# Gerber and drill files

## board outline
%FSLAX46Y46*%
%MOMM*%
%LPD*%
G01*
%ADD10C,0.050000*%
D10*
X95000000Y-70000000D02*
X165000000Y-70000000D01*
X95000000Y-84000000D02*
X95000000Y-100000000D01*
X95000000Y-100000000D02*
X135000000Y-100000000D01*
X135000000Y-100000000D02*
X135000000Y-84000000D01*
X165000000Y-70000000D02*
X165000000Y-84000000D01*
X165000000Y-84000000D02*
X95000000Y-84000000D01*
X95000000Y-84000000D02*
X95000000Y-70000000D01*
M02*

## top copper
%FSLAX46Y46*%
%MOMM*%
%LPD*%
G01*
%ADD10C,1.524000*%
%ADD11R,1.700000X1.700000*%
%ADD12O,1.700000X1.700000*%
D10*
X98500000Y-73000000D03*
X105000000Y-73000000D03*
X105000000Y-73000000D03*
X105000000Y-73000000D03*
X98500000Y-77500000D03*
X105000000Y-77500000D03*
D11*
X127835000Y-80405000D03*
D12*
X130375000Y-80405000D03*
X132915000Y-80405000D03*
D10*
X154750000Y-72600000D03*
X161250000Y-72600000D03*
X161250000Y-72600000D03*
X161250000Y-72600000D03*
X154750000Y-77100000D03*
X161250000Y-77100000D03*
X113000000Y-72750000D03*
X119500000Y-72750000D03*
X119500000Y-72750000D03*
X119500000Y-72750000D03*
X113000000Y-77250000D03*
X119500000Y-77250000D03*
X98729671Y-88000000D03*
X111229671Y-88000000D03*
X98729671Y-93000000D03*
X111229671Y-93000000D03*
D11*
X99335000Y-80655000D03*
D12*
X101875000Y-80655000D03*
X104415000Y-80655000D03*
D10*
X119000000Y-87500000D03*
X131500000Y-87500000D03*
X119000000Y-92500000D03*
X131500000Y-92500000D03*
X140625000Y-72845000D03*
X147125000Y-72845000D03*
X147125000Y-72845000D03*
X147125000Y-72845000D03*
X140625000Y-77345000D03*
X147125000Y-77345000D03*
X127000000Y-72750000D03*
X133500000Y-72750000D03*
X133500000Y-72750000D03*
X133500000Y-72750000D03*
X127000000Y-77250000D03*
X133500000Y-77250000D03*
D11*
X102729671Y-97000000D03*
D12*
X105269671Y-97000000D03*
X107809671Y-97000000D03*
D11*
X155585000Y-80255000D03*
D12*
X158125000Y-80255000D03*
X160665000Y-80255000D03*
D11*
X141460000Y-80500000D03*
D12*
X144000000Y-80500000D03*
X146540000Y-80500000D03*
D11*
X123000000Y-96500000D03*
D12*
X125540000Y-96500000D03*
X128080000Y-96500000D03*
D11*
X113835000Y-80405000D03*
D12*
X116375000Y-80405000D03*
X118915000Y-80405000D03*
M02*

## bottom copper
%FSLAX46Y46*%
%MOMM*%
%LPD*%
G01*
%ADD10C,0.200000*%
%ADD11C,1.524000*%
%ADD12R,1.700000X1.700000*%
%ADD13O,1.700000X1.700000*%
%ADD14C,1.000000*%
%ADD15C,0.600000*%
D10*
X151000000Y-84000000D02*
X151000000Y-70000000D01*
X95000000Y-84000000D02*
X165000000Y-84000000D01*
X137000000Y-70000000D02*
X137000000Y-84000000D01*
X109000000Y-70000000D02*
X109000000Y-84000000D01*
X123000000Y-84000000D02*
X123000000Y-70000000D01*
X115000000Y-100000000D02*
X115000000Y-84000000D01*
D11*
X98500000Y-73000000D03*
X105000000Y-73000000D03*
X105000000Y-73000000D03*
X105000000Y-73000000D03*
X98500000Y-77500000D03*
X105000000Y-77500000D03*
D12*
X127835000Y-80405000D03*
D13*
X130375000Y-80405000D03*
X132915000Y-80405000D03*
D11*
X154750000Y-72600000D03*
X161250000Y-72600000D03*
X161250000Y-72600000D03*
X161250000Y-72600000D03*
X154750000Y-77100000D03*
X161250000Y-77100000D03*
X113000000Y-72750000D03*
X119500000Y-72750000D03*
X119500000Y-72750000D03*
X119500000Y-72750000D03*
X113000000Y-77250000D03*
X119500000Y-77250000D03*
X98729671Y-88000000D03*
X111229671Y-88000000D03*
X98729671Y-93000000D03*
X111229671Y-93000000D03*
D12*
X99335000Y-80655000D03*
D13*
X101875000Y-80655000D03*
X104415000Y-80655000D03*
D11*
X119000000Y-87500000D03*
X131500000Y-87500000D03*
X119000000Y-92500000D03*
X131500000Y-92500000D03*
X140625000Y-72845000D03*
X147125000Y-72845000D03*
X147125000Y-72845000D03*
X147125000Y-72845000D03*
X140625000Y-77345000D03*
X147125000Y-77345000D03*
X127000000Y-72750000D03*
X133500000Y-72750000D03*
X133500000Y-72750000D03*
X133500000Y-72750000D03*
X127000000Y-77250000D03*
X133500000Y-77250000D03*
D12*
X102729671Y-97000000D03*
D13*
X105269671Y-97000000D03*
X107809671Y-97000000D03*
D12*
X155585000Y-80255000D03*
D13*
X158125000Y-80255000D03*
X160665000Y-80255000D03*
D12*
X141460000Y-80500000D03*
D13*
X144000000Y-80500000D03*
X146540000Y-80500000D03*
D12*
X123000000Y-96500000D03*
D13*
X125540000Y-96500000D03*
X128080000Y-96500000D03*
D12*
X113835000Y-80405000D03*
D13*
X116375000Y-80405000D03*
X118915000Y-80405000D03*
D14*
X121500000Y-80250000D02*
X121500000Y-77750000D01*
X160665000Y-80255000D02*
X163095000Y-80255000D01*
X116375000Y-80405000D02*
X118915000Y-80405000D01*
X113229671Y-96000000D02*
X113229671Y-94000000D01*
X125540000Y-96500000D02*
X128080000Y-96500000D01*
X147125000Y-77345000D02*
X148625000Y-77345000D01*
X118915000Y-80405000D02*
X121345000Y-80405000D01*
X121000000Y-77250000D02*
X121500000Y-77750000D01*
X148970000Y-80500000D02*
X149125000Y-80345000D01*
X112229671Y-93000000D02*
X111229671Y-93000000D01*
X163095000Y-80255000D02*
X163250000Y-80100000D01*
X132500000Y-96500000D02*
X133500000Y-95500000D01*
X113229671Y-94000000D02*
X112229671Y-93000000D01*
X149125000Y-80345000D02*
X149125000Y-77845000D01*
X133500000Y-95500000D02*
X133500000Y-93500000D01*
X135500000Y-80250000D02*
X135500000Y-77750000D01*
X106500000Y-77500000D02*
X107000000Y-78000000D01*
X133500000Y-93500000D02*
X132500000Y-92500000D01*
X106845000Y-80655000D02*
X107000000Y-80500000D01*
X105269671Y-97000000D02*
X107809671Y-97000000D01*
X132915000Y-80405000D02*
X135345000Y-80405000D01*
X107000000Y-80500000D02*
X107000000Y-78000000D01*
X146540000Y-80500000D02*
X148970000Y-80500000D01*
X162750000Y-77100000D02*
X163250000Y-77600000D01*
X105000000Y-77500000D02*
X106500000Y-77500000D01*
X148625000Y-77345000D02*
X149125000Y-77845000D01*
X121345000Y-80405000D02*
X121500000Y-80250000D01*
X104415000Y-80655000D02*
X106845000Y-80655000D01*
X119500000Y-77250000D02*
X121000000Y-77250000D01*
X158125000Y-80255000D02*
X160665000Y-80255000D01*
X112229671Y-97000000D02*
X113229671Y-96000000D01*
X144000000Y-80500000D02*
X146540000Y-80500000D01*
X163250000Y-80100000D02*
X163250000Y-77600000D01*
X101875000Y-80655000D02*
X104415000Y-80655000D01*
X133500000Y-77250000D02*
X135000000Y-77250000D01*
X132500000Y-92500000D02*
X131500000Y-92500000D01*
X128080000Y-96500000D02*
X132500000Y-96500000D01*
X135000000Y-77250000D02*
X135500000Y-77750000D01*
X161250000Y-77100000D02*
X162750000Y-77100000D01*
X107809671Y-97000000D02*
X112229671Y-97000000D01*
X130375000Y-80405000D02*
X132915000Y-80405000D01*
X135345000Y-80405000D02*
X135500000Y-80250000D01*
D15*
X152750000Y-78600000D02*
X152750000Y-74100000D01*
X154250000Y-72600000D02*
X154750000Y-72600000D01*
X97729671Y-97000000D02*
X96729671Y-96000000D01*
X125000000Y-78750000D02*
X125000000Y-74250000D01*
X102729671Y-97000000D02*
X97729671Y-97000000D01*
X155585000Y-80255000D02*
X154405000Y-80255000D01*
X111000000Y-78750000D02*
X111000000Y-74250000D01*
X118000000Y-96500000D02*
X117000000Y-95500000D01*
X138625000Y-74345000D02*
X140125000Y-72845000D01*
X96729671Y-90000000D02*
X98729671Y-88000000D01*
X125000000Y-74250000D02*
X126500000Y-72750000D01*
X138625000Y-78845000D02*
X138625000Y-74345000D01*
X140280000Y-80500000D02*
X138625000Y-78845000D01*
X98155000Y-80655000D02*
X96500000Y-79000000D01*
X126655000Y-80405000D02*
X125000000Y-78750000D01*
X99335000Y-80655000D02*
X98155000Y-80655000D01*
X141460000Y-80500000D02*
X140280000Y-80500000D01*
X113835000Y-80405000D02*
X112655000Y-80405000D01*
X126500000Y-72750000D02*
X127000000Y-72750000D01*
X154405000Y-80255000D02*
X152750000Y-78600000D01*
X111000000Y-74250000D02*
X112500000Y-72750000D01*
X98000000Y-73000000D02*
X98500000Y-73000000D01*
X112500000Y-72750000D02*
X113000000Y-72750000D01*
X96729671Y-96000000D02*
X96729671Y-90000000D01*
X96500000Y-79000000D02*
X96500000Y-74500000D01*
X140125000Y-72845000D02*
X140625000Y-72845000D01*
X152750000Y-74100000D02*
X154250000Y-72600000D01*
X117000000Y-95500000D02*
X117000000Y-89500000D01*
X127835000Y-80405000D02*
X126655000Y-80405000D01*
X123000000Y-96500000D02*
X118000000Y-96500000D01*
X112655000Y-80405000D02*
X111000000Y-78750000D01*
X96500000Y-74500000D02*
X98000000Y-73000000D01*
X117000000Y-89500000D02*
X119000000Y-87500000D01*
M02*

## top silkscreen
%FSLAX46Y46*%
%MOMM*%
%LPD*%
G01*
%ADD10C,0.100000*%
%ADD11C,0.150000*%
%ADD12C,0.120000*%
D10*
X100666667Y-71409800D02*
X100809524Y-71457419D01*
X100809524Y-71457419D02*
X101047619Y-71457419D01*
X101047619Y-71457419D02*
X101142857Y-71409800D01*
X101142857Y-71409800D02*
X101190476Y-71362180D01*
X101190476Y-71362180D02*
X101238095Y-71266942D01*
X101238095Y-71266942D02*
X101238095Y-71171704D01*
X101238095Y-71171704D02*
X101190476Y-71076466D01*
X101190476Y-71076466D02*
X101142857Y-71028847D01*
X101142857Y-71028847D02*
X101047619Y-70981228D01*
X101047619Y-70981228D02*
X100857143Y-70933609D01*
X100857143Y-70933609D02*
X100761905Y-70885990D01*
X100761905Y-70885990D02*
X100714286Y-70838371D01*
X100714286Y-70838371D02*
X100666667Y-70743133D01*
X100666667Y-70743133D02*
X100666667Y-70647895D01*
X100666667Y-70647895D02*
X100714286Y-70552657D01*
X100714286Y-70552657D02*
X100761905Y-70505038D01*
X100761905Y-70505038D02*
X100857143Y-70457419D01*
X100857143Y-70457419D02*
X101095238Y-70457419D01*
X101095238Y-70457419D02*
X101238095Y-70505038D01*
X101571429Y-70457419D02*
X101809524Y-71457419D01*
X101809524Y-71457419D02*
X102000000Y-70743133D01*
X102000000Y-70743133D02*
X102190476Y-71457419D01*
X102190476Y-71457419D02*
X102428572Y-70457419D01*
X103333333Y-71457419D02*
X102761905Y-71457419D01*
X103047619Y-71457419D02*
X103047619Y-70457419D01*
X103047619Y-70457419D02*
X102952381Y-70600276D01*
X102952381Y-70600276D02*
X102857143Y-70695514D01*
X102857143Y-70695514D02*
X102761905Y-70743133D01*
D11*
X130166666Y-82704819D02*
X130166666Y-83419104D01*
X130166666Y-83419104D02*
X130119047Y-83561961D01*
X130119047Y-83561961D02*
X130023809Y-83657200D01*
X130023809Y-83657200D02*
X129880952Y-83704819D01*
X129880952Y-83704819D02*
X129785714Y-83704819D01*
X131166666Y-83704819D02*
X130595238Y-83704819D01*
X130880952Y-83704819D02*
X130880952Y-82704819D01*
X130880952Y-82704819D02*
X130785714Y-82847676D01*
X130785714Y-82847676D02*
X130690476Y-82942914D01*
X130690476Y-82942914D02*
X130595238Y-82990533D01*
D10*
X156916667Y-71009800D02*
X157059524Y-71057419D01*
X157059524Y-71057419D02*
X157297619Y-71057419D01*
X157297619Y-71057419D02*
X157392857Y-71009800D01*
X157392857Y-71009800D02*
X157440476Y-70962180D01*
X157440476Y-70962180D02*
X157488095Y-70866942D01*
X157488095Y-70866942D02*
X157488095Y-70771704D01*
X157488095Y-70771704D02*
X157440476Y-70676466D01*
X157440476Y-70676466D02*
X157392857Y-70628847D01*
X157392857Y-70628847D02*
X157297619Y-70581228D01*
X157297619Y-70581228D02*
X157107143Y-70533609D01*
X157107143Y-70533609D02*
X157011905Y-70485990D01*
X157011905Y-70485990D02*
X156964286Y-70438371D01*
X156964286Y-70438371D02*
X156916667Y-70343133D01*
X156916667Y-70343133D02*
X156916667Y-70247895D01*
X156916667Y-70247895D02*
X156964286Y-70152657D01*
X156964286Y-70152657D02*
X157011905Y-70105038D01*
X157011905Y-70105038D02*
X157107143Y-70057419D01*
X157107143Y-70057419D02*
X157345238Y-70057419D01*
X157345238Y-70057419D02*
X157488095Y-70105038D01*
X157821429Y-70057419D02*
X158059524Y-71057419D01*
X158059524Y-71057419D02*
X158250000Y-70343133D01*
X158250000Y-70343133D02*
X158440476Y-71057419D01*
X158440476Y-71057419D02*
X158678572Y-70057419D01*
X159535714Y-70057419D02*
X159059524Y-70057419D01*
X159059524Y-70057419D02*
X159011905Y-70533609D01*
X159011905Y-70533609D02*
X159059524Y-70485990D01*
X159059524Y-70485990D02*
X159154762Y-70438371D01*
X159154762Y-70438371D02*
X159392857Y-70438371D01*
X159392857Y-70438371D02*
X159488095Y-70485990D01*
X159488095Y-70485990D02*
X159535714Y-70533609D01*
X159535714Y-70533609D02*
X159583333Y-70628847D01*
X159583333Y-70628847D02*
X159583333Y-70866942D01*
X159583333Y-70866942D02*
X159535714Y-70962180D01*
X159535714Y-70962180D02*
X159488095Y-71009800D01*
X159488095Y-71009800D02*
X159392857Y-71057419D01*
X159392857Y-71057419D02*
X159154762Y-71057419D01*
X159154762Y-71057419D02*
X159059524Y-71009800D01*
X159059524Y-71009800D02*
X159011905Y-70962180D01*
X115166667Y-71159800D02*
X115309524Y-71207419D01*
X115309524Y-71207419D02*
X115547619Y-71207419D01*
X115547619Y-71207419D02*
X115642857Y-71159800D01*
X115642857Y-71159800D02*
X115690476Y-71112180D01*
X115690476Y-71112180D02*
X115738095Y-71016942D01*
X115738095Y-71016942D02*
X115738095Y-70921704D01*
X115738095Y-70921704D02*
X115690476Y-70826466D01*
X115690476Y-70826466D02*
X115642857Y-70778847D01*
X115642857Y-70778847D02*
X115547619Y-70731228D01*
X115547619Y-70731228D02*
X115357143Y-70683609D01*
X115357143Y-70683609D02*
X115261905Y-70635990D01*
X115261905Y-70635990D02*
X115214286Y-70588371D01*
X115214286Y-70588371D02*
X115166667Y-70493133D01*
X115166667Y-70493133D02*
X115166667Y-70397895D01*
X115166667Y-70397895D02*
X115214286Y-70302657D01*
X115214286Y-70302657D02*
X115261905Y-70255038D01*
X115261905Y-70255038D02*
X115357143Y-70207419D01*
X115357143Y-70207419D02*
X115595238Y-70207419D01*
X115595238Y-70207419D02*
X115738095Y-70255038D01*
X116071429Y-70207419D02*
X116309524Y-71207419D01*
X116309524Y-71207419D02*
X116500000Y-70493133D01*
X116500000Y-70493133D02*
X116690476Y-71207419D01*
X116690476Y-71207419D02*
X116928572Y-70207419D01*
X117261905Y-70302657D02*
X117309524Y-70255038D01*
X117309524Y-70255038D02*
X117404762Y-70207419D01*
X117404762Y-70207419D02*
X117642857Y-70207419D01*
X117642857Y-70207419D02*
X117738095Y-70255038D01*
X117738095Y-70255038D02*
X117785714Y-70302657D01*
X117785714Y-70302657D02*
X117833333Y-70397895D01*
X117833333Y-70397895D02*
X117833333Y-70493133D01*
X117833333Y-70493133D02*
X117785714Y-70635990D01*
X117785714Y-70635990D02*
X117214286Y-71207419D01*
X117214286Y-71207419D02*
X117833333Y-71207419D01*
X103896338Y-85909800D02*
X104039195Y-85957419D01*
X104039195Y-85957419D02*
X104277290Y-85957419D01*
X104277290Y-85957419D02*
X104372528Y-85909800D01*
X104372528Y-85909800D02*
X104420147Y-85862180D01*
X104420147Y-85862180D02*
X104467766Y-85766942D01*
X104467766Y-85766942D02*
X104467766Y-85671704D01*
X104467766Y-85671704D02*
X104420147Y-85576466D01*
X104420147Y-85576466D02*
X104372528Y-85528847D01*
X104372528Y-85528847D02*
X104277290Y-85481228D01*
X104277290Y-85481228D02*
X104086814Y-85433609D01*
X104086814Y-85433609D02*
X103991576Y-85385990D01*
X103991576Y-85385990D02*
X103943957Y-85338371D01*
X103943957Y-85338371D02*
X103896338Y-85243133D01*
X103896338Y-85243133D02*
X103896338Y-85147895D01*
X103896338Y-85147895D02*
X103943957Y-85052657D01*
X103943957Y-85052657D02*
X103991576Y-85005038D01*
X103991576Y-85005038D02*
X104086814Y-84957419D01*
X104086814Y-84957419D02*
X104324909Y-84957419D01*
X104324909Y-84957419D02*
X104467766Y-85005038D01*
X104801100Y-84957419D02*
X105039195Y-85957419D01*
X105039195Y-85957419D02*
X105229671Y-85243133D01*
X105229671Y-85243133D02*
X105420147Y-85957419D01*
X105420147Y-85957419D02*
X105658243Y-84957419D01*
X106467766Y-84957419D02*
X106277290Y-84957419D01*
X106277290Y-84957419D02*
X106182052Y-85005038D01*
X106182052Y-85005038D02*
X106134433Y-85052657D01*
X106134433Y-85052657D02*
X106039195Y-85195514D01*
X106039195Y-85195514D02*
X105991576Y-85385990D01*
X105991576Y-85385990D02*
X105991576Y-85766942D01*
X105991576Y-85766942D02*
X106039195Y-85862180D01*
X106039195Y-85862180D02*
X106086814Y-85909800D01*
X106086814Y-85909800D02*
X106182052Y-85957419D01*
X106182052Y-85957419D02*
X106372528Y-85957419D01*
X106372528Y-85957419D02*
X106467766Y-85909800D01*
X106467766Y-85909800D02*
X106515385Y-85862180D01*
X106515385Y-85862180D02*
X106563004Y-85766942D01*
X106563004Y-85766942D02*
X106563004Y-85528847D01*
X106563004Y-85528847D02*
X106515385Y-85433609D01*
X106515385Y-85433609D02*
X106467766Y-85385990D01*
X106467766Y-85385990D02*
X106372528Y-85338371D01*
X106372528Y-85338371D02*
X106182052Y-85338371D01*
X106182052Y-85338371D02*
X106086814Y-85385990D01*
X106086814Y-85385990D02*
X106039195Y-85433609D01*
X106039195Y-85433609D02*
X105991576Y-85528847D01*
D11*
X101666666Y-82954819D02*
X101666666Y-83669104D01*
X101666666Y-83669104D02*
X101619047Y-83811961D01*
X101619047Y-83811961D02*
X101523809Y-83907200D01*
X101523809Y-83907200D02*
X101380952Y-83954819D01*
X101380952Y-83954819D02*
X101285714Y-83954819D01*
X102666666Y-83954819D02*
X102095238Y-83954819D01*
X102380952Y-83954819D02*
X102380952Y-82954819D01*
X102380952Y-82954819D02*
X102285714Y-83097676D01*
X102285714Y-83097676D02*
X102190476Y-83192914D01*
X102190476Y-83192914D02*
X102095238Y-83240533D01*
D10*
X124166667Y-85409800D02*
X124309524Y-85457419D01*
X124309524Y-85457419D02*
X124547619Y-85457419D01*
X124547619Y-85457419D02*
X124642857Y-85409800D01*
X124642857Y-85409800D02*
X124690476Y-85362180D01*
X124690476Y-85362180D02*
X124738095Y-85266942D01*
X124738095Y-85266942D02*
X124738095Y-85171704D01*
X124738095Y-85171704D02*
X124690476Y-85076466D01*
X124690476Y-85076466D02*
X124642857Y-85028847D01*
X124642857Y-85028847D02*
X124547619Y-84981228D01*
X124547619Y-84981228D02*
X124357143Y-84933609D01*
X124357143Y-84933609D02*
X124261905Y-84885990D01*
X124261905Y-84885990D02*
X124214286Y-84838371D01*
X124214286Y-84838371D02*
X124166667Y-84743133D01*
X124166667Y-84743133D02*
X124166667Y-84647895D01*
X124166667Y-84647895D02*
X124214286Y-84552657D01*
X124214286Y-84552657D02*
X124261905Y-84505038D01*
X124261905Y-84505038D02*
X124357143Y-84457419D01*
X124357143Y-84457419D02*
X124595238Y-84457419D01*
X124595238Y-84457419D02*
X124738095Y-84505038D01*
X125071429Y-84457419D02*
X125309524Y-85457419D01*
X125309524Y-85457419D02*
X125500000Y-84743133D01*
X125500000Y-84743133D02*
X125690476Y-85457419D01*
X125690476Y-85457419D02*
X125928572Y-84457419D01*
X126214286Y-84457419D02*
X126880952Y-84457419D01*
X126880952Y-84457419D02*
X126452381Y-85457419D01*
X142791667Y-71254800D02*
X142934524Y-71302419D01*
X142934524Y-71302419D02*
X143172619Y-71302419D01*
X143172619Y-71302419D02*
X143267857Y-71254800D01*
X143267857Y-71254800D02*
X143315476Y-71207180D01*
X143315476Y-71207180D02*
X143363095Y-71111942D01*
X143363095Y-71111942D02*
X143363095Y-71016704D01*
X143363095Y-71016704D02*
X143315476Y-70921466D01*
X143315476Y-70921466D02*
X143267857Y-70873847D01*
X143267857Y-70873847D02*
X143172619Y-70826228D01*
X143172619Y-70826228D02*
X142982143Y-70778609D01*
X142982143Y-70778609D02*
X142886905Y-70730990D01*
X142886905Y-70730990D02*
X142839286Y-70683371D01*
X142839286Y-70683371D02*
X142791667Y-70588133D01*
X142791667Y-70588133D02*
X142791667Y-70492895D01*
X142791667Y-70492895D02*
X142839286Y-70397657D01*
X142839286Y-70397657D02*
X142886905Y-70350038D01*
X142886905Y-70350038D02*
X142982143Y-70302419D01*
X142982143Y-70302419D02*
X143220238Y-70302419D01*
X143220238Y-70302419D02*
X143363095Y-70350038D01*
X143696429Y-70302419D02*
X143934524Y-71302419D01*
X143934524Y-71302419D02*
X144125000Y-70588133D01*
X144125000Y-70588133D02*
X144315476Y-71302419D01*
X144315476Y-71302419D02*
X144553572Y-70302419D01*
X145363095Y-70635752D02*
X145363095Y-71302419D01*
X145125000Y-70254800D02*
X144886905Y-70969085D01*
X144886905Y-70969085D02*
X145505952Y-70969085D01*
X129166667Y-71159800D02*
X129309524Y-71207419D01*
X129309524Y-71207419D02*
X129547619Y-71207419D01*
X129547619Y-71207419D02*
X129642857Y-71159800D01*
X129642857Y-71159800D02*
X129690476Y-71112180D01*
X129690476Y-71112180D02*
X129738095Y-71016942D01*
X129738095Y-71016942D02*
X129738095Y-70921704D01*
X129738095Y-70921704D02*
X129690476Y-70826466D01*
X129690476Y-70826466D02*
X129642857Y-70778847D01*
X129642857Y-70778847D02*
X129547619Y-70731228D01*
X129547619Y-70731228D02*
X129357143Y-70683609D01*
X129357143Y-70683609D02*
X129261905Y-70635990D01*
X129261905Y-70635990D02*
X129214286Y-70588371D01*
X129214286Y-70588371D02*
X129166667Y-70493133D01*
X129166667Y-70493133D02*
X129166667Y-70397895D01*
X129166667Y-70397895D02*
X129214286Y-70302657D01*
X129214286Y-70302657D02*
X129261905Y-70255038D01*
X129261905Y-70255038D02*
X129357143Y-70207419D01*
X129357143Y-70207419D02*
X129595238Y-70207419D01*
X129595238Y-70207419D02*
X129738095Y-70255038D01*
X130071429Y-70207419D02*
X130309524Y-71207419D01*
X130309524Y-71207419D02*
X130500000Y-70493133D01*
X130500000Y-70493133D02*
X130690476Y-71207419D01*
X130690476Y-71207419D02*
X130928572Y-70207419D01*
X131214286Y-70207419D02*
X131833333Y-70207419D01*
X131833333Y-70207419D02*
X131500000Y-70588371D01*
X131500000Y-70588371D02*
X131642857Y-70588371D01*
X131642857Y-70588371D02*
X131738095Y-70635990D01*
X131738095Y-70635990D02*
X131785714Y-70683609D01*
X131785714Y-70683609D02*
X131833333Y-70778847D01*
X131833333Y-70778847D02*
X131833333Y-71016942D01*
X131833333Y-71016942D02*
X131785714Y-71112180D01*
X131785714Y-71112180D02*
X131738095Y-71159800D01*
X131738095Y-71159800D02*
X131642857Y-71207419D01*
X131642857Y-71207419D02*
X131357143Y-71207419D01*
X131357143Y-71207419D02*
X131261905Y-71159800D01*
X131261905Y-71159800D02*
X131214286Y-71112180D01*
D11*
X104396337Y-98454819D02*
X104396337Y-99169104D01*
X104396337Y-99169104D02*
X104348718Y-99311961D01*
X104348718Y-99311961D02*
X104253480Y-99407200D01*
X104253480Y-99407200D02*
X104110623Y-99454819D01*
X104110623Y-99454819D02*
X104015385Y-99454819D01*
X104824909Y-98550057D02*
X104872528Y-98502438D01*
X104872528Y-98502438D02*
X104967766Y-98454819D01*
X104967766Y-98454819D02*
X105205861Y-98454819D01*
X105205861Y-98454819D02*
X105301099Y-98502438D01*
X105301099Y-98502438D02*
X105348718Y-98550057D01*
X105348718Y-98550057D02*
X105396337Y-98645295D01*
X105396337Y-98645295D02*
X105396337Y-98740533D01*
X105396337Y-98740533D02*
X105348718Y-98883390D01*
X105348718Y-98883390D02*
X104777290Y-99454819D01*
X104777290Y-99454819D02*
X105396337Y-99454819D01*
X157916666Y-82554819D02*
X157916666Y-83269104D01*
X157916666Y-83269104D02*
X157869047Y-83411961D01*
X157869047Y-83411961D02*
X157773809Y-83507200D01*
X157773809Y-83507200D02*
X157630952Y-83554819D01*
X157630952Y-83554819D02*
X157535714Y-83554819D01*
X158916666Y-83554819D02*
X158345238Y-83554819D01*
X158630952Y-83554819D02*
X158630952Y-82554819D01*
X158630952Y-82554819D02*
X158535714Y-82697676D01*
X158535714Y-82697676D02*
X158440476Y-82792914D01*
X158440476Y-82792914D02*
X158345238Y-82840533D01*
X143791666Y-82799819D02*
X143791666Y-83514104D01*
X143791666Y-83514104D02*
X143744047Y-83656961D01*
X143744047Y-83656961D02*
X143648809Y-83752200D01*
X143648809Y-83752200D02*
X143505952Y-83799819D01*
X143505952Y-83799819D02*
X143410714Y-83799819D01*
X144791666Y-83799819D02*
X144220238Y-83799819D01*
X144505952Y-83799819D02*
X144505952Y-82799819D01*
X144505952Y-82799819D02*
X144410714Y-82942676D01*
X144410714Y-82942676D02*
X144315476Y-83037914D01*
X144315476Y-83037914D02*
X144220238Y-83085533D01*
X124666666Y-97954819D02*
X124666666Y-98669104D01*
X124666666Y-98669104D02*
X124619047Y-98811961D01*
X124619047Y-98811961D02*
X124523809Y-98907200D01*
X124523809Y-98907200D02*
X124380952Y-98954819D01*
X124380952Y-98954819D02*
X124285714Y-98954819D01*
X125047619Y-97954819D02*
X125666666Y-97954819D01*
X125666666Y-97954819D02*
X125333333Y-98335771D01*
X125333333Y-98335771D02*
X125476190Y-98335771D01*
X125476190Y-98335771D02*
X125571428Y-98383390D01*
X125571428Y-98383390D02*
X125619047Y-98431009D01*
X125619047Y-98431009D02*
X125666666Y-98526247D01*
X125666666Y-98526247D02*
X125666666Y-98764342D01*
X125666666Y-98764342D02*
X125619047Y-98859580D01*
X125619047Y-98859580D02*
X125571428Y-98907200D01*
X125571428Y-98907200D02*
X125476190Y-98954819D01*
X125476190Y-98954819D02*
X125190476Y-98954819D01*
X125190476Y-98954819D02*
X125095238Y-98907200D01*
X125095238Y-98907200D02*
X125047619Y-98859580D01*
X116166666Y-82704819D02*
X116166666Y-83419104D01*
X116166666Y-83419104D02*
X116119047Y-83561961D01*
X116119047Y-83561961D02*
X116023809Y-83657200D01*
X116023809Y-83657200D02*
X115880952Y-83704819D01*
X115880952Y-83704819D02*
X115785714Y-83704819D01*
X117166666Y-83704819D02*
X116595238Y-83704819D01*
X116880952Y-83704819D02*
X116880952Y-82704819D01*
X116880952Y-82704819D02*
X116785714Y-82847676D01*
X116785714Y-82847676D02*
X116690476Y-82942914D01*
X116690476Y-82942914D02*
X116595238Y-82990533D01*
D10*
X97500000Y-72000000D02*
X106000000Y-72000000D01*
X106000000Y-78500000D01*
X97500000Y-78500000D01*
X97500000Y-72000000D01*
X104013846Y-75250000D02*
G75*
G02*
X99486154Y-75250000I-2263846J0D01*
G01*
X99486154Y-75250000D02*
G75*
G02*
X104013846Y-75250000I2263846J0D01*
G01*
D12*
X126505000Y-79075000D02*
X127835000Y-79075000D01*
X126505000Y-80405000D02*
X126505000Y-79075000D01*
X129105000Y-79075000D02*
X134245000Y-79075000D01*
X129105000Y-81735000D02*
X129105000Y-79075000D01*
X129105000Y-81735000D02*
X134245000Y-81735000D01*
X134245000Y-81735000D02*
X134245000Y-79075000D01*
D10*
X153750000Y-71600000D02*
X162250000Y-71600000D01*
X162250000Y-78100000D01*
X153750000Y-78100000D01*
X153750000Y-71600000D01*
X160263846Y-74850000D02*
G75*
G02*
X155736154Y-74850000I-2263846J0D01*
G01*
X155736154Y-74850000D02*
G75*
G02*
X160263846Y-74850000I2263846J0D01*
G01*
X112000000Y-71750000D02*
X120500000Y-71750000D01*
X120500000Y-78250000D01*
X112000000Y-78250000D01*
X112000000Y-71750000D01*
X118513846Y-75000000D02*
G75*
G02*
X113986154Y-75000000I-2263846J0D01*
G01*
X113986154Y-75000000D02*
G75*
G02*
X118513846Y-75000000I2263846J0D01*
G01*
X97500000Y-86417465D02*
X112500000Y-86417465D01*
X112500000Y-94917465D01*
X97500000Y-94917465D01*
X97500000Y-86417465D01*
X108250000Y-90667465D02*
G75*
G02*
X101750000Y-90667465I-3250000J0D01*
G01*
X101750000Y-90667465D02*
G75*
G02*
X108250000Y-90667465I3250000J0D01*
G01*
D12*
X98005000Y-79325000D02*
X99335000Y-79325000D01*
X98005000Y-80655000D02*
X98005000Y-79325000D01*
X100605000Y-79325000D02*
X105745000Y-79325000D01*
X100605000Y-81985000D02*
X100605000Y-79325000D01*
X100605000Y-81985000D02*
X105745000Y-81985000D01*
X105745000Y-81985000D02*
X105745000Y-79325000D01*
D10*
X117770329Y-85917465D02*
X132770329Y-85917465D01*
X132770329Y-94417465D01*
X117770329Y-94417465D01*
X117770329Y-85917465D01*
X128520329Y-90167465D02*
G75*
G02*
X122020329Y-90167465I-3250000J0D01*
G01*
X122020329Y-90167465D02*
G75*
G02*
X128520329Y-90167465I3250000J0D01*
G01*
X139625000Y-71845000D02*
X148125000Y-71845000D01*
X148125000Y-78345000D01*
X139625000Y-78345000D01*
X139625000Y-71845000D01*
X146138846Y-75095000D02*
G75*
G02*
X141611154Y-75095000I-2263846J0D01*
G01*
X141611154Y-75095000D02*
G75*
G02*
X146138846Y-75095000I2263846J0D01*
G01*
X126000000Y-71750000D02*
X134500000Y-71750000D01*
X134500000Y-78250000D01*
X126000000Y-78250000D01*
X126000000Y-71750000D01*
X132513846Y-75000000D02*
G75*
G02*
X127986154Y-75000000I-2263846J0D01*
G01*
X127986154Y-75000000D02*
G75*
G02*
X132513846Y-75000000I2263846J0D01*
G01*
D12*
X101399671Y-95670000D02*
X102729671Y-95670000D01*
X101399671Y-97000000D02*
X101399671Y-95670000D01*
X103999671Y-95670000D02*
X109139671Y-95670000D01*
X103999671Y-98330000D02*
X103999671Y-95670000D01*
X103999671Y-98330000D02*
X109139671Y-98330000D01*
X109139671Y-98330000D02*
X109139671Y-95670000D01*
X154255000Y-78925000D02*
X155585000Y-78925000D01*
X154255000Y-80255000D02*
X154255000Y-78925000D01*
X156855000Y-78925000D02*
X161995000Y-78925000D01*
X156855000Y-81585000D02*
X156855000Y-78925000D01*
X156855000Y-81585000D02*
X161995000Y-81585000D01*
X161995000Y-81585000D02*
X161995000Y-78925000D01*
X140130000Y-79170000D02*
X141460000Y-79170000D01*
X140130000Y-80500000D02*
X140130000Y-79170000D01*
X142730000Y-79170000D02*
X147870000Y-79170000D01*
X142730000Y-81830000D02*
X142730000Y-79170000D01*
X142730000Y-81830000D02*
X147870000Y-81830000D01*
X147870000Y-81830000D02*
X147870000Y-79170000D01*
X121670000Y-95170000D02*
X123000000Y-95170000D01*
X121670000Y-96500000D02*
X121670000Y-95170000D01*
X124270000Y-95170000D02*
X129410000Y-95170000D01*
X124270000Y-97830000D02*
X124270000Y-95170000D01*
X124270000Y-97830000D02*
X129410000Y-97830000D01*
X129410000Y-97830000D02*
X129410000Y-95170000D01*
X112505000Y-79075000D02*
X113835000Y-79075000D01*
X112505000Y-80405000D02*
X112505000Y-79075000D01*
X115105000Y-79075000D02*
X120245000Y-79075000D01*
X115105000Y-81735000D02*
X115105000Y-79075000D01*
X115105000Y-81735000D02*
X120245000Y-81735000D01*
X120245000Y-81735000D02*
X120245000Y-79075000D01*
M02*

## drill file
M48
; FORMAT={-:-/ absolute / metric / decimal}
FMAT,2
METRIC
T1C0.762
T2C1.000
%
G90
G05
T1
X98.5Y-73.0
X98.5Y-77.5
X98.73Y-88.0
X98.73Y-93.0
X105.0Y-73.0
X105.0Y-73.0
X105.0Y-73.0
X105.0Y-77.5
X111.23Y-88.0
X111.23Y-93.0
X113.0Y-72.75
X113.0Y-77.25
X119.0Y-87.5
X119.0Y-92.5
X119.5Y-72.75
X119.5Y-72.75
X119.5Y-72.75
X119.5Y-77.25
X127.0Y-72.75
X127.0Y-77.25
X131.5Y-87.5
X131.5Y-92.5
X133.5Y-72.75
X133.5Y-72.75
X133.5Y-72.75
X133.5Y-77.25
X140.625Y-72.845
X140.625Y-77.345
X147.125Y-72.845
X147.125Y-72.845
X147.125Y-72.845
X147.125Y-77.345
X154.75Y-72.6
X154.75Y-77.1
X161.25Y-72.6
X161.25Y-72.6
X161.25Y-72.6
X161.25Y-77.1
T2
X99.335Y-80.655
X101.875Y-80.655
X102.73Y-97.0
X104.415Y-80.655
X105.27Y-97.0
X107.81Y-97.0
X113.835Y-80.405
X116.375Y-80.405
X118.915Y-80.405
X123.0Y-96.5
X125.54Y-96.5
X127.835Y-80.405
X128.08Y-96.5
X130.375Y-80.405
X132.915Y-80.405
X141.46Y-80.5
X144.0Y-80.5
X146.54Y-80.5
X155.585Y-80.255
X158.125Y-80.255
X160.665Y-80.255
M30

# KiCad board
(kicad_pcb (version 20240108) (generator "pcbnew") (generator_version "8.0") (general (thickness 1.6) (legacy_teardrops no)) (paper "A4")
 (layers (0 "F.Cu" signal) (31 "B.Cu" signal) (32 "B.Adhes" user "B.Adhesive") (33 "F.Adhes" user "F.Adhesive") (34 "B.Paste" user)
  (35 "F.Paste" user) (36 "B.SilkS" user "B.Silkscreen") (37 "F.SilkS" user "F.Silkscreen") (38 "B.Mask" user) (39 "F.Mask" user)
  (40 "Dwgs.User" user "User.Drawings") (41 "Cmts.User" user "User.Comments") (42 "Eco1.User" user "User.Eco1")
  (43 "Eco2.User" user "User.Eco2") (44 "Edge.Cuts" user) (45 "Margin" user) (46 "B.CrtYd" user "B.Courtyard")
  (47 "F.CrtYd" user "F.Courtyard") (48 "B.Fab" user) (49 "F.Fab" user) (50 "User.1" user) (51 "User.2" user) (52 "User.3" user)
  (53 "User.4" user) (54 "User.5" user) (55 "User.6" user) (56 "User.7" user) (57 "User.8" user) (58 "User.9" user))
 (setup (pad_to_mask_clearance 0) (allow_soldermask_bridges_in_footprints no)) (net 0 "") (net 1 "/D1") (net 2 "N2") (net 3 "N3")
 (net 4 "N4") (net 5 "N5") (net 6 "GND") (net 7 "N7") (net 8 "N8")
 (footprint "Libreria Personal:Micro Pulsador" (layer "F.Cu") (at 102.5 66.5)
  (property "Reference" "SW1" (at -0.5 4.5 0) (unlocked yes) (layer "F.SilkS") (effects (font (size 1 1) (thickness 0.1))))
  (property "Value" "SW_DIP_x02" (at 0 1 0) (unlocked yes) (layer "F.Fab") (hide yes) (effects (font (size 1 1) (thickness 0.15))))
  (fp_rect (start -5 5.5) (end 3.5 12) (stroke (width 0.1) (type default)) (fill none) (layer "F.SilkS"))
  (fp_circle (center -0.75 8.75) (end 1.5 8.5) (stroke (width 0.1) (type default)) (fill none) (layer "F.SilkS"))
  (pad "1" thru_hole circle (at -4 6.5) (size 1.524 1.524) (drill 0.762) (layers "*.Cu" "*.Mask") (remove_unused_layers no) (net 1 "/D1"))
  (pad "2" thru_hole circle (at 2.5 6.5) (size 1.524 1.524) (drill 0.762) (layers "*.Cu" "*.Mask") (remove_unused_layers no) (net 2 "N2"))
  (pad "2" thru_hole circle (at 2.5 6.5) (size 1.524 1.524) (drill 0.762) (layers "*.Cu" "*.Mask") (remove_unused_layers no) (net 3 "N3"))
  (pad "2" thru_hole circle (at 2.5 6.5) (size 1.524 1.524) (drill 0.762) (layers "*.Cu" "*.Mask") (remove_unused_layers no) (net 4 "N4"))
  (pad "3" thru_hole circle (at -4 11) (size 1.524 1.524) (drill 0.762) (layers "*.Cu" "*.Mask") (remove_unused_layers no) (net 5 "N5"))
  (pad "4" thru_hole circle (at 2.5 11) (size 1.524 1.524) (drill 0.762) (layers "*.Cu" "*.Mask") (remove_unused_layers no) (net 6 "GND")))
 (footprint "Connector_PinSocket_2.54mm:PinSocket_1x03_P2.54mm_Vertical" (layer "F.Cu") (at 127.835 80.405 90)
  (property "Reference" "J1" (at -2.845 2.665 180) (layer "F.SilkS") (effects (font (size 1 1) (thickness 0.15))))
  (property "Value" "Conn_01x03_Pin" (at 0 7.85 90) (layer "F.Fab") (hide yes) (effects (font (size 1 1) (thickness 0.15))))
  (fp_line (start 1.33 -1.33) (end 1.33 0) (stroke (width 0.12) (type solid)) (layer "F.SilkS"))
  (fp_line (start 0 -1.33) (end 1.33 -1.33) (stroke (width 0.12) (type solid)) (layer "F.SilkS"))
  (fp_line (start 1.33 1.27) (end 1.33 6.41) (stroke (width 0.12) (type solid)) (layer "F.SilkS"))
  (fp_line (start -1.33 1.27) (end 1.33 1.27) (stroke (width 0.12) (type solid)) (layer "F.SilkS"))
  (fp_line (start -1.33 1.27) (end -1.33 6.41) (stroke (width 0.12) (type solid)) (layer "F.SilkS"))
  (fp_line (start -1.33 6.41) (end 1.33 6.41) (stroke (width 0.12) (type solid)) (layer "F.SilkS"))
  (pad "1" thru_hole rect (at 0 0 90) (size 1.7 1.7) (drill 1) (layers "*.Cu" "*.Mask") (remove_unused_layers no) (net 1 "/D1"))
  (pad "2" thru_hole oval (at 0 2.54 90) (size 1.7 1.7) (drill 1) (layers "*.Cu" "*.Mask") (remove_unused_layers no) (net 6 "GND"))
  (pad "3" thru_hole oval (at 0 5.08 90) (size 1.7 1.7) (drill 1) (layers "*.Cu" "*.Mask") (remove_unused_layers no) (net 6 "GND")))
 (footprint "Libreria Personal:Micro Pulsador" (layer "F.Cu") (at 158.75 66.1)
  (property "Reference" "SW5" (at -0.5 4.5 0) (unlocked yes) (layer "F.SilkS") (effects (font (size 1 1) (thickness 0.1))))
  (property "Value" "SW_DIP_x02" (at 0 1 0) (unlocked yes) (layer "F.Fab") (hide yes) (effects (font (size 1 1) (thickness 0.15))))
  (fp_rect (start -5 5.5) (end 3.5 12) (stroke (width 0.1) (type default)) (fill none) (layer "F.SilkS"))
  (fp_circle (center -0.75 8.75) (end 1.5 8.5) (stroke (width 0.1) (type default)) (fill none) (layer "F.SilkS"))
  (pad "1" thru_hole circle (at -4 6.5) (size 1.524 1.524) (drill 0.762) (layers "*.Cu" "*.Mask") (remove_unused_layers no) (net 1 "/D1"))
  (pad "2" thru_hole circle (at 2.5 6.5) (size 1.524 1.524) (drill 0.762) (layers "*.Cu" "*.Mask") (remove_unused_layers no) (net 2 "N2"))
  (pad "2" thru_hole circle (at 2.5 6.5) (size 1.524 1.524) (drill 0.762) (layers "*.Cu" "*.Mask") (remove_unused_layers no) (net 3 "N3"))
  (pad "2" thru_hole circle (at 2.5 6.5) (size 1.524 1.524) (drill 0.762) (layers "*.Cu" "*.Mask") (remove_unused_layers no) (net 4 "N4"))
  (pad "3" thru_hole circle (at -4 11) (size 1.524 1.524) (drill 0.762) (layers "*.Cu" "*.Mask") (remove_unused_layers no) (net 5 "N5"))
  (pad "4" thru_hole circle (at 2.5 11) (size 1.524 1.524) (drill 0.762) (layers "*.Cu" "*.Mask") (remove_unused_layers no) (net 6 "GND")))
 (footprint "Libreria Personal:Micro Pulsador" (layer "F.Cu") (at 117 66.25)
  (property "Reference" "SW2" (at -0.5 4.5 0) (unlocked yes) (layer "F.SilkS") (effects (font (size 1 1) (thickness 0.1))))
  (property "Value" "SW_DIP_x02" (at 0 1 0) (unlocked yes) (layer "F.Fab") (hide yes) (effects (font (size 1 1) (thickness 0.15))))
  (fp_rect (start -5 5.5) (end 3.5 12) (stroke (width 0.1) (type default)) (fill none) (layer "F.SilkS"))
  (fp_circle (center -0.75 8.75) (end 1.5 8.5) (stroke (width 0.1) (type default)) (fill none) (layer "F.SilkS"))
  (pad "1" thru_hole circle (at -4 6.5) (size 1.524 1.524) (drill 0.762) (layers "*.Cu" "*.Mask") (remove_unused_layers no) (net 1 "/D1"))
  (pad "2" thru_hole circle (at 2.5 6.5) (size 1.524 1.524) (drill 0.762) (layers "*.Cu" "*.Mask") (remove_unused_layers no) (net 2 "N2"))
  (pad "2" thru_hole circle (at 2.5 6.5) (size 1.524 1.524) (drill 0.762) (layers "*.Cu" "*.Mask") (remove_unused_layers no) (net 3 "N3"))
  (pad "2" thru_hole circle (at 2.5 6.5) (size 1.524 1.524) (drill 0.762) (layers "*.Cu" "*.Mask") (remove_unused_layers no) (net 4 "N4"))
  (pad "3" thru_hole circle (at -4 11) (size 1.524 1.524) (drill 0.762) (layers "*.Cu" "*.Mask") (remove_unused_layers no) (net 5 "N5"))
  (pad "4" thru_hole circle (at 2.5 11) (size 1.524 1.524) (drill 0.762) (layers "*.Cu" "*.Mask") (remove_unused_layers no) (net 6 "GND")))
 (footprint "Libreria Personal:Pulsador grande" (layer "F.Cu") (at 102.5 81.917465)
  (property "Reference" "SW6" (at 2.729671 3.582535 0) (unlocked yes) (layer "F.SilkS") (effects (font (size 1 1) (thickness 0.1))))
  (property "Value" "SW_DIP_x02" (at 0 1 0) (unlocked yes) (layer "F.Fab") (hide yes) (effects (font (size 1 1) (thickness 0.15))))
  (fp_rect (start -5 4.5) (end 10 13) (stroke (width 0.1) (type default)) (fill none) (layer "F.SilkS"))
  (fp_circle (center 2.5 8.75) (end 5.5 7.5) (stroke (width 0.1) (type default)) (fill none) (layer "F.SilkS"))
  (pad "1" thru_hole circle (at -3.770329 6.082535) (size 1.524 1.524) (drill 0.762) (layers "*.Cu" "*.Mask") (remove_unused_layers no)
   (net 1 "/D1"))
  (pad "2" thru_hole circle (at 8.729671 6.082535) (size 1.524 1.524) (drill 0.762) (layers "*.Cu" "*.Mask") (remove_unused_layers no)
   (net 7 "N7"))
  (pad "3" thru_hole circle (at -3.770329 11.082535) (size 1.524 1.524) (drill 0.762) (layers "*.Cu" "*.Mask") (remove_unused_layers no)
   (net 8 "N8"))
  (pad "4" thru_hole circle (at 8.729671 11.082535) (size 1.524 1.524) (drill 0.762) (layers "*.Cu" "*.Mask") (remove_unused_layers no)
   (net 6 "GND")))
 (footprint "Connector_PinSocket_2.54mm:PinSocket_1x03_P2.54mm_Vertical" (layer "F.Cu") (at 99.335 80.655 90)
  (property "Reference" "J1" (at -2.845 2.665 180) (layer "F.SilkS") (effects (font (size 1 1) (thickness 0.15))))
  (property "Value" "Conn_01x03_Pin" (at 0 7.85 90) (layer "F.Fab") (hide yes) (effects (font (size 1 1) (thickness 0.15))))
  (fp_line (start 1.33 -1.33) (end 1.33 0) (stroke (width 0.12) (type solid)) (layer "F.SilkS"))
  (fp_line (start 0 -1.33) (end 1.33 -1.33) (stroke (width 0.12) (type solid)) (layer "F.SilkS"))
  (fp_line (start 1.33 1.27) (end 1.33 6.41) (stroke (width 0.12) (type solid)) (layer "F.SilkS"))
  (fp_line (start -1.33 1.27) (end 1.33 1.27) (stroke (width 0.12) (type solid)) (layer "F.SilkS"))
  (fp_line (start -1.33 1.27) (end -1.33 6.41) (stroke (width 0.12) (type solid)) (layer "F.SilkS"))
  (fp_line (start -1.33 6.41) (end 1.33 6.41) (stroke (width 0.12) (type solid)) (layer "F.SilkS"))
  (pad "1" thru_hole rect (at 0 0 90) (size 1.7 1.7) (drill 1) (layers "*.Cu" "*.Mask") (remove_unused_layers no) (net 1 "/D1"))
  (pad "2" thru_hole oval (at 0 2.54 90) (size 1.7 1.7) (drill 1) (layers "*.Cu" "*.Mask") (remove_unused_layers no) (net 6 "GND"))
  (pad "3" thru_hole oval (at 0 5.08 90) (size 1.7 1.7) (drill 1) (layers "*.Cu" "*.Mask") (remove_unused_layers no) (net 6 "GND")))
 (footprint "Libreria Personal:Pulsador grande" (layer "F.Cu") (at 122.770329 81.417465)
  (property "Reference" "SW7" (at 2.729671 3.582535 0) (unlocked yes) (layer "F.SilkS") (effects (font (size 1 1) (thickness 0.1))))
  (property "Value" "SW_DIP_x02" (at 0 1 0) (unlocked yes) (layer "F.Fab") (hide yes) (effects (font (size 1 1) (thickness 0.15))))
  (fp_rect (start -5 4.5) (end 10 13) (stroke (width 0.1) (type default)) (fill none) (layer "F.SilkS"))
  (fp_circle (center 2.5 8.75) (end 5.5 7.5) (stroke (width 0.1) (type default)) (fill none) (layer "F.SilkS"))
  (pad "1" thru_hole circle (at -3.770329 6.082535) (size 1.524 1.524) (drill 0.762) (layers "*.Cu" "*.Mask") (remove_unused_layers no)
   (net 1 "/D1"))
  (pad "2" thru_hole circle (at 8.729671 6.082535) (size 1.524 1.524) (drill 0.762) (layers "*.Cu" "*.Mask") (remove_unused_layers no)
   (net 7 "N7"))
  (pad "3" thru_hole circle (at -3.770329 11.082535) (size 1.524 1.524) (drill 0.762) (layers "*.Cu" "*.Mask") (remove_unused_layers no)
   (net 8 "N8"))
  (pad "4" thru_hole circle (at 8.729671 11.082535) (size 1.524 1.524) (drill 0.762) (layers "*.Cu" "*.Mask") (remove_unused_layers no)
   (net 6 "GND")))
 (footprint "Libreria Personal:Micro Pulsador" (layer "F.Cu") (at 144.625 66.345)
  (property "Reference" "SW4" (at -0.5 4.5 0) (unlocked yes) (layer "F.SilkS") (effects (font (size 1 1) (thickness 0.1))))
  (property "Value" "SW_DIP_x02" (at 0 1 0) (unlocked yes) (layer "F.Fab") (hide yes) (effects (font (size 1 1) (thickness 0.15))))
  (fp_rect (start -5 5.5) (end 3.5 12) (stroke (width 0.1) (type default)) (fill none) (layer "F.SilkS"))
  (fp_circle (center -0.75 8.75) (end 1.5 8.5) (stroke (width 0.1) (type default)) (fill none) (layer "F.SilkS"))
  (pad "1" thru_hole circle (at -4 6.5) (size 1.524 1.524) (drill 0.762) (layers "*.Cu" "*.Mask") (remove_unused_layers no) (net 1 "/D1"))
  (pad "2" thru_hole circle (at 2.5 6.5) (size 1.524 1.524) (drill 0.762) (layers "*.Cu" "*.Mask") (remove_unused_layers no) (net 2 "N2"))
  (pad "2" thru_hole circle (at 2.5 6.5) (size 1.524 1.524) (drill 0.762) (layers "*.Cu" "*.Mask") (remove_unused_layers no) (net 3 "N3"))
  (pad "2" thru_hole circle (at 2.5 6.5) (size 1.524 1.524) (drill 0.762) (layers "*.Cu" "*.Mask") (remove_unused_layers no) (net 4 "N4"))
  (pad "3" thru_hole circle (at -4 11) (size 1.524 1.524) (drill 0.762) (layers "*.Cu" "*.Mask") (remove_unused_layers no) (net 5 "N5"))
  (pad "4" thru_hole circle (at 2.5 11) (size 1.524 1.524) (drill 0.762) (layers "*.Cu" "*.Mask") (remove_unused_layers no) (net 6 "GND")))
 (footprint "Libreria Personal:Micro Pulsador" (layer "F.Cu") (at 131 66.25)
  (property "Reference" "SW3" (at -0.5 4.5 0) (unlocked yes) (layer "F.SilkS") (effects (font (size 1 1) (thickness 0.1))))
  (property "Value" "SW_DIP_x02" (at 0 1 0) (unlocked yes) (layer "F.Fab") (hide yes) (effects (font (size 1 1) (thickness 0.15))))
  (fp_rect (start -5 5.5) (end 3.5 12) (stroke (width 0.1) (type default)) (fill none) (layer "F.SilkS"))
  (fp_circle (center -0.75 8.75) (end 1.5 8.5) (stroke (width 0.1) (type default)) (fill none) (layer "F.SilkS"))
  (pad "1" thru_hole circle (at -4 6.5) (size 1.524 1.524) (drill 0.762) (layers "*.Cu" "*.Mask") (remove_unused_layers no) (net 1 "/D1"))
  (pad "2" thru_hole circle (at 2.5 6.5) (size 1.524 1.524) (drill 0.762) (layers "*.Cu" "*.Mask") (remove_unused_layers no) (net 2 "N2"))
  (pad "2" thru_hole circle (at 2.5 6.5) (size 1.524 1.524) (drill 0.762) (layers "*.Cu" "*.Mask") (remove_unused_layers no) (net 3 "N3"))
  (pad "2" thru_hole circle (at 2.5 6.5) (size 1.524 1.524) (drill 0.762) (layers "*.Cu" "*.Mask") (remove_unused_layers no) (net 4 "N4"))
  (pad "3" thru_hole circle (at -4 11) (size 1.524 1.524) (drill 0.762) (layers "*.Cu" "*.Mask") (remove_unused_layers no) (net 5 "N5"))
  (pad "4" thru_hole circle (at 2.5 11) (size 1.524 1.524) (drill 0.762) (layers "*.Cu" "*.Mask") (remove_unused_layers no) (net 6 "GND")))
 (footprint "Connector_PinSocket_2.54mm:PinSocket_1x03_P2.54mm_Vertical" (layer "F.Cu") (at 102.729671 97 90)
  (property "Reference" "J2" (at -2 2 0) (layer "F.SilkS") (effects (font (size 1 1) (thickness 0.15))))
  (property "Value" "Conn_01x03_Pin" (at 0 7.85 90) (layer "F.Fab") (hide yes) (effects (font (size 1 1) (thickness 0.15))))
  (fp_line (start 1.33 -1.33) (end 1.33 0) (stroke (width 0.12) (type solid)) (layer "F.SilkS"))
  (fp_line (start 0 -1.33) (end 1.33 -1.33) (stroke (width 0.12) (type solid)) (layer "F.SilkS"))
  (fp_line (start 1.33 1.27) (end 1.33 6.41) (stroke (width 0.12) (type solid)) (layer "F.SilkS"))
  (fp_line (start -1.33 1.27) (end 1.33 1.27) (stroke (width 0.12) (type solid)) (layer "F.SilkS"))
  (fp_line (start -1.33 1.27) (end -1.33 6.41) (stroke (width 0.12) (type solid)) (layer "F.SilkS"))
  (fp_line (start -1.33 6.41) (end 1.33 6.41) (stroke (width 0.12) (type solid)) (layer "F.SilkS"))
  (pad "1" thru_hole rect (at 0 0 90) (size 1.7 1.7) (drill 1) (layers "*.Cu" "*.Mask") (remove_unused_layers no) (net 1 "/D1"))
  (pad "2" thru_hole oval (at 0 2.54 90) (size 1.7 1.7) (drill 1) (layers "*.Cu" "*.Mask") (remove_unused_layers no) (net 6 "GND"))
  (pad "3" thru_hole oval (at 0 5.08 90) (size 1.7 1.7) (drill 1) (layers "*.Cu" "*.Mask") (remove_unused_layers no) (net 6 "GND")))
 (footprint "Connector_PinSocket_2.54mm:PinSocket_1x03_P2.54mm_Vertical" (layer "F.Cu") (at 155.585 80.255 90)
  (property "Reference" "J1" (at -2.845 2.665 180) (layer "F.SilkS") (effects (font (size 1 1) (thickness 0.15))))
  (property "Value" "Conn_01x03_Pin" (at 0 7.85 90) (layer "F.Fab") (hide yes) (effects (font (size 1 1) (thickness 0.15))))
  (fp_line (start 1.33 -1.33) (end 1.33 0) (stroke (width 0.12) (type solid)) (layer "F.SilkS"))
  (fp_line (start 0 -1.33) (end 1.33 -1.33) (stroke (width 0.12) (type solid)) (layer "F.SilkS"))
  (fp_line (start 1.33 1.27) (end 1.33 6.41) (stroke (width 0.12) (type solid)) (layer "F.SilkS"))
  (fp_line (start -1.33 1.27) (end 1.33 1.27) (stroke (width 0.12) (type solid)) (layer "F.SilkS"))
  (fp_line (start -1.33 1.27) (end -1.33 6.41) (stroke (width 0.12) (type solid)) (layer "F.SilkS"))
  (fp_line (start -1.33 6.41) (end 1.33 6.41) (stroke (width 0.12) (type solid)) (layer "F.SilkS"))
  (pad "1" thru_hole rect (at 0 0 90) (size 1.7 1.7) (drill 1) (layers "*.Cu" "*.Mask") (remove_unused_layers no) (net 1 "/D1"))
  (pad "2" thru_hole oval (at 0 2.54 90) (size 1.7 1.7) (drill 1) (layers "*.Cu" "*.Mask") (remove_unused_layers no) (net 6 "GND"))
  (pad "3" thru_hole oval (at 0 5.08 90) (size 1.7 1.7) (drill 1) (layers "*.Cu" "*.Mask") (remove_unused_layers no) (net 6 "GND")))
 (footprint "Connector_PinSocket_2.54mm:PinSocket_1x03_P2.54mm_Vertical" (layer "F.Cu") (at 141.46 80.5 90)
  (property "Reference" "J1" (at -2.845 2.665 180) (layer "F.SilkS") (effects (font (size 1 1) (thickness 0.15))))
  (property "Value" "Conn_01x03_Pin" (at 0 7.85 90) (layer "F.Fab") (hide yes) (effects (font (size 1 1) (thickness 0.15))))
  (fp_line (start 1.33 -1.33) (end 1.33 0) (stroke (width 0.12) (type solid)) (layer "F.SilkS"))
  (fp_line (start 0 -1.33) (end 1.33 -1.33) (stroke (width 0.12) (type solid)) (layer "F.SilkS"))
  (fp_line (start 1.33 1.27) (end 1.33 6.41) (stroke (width 0.12) (type solid)) (layer "F.SilkS"))
  (fp_line (start -1.33 1.27) (end 1.33 1.27) (stroke (width 0.12) (type solid)) (layer "F.SilkS"))
  (fp_line (start -1.33 1.27) (end -1.33 6.41) (stroke (width 0.12) (type solid)) (layer "F.SilkS"))
  (fp_line (start -1.33 6.41) (end 1.33 6.41) (stroke (width 0.12) (type solid)) (layer "F.SilkS"))
  (pad "1" thru_hole rect (at 0 0 90) (size 1.7 1.7) (drill 1) (layers "*.Cu" "*.Mask") (remove_unused_layers no) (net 1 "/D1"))
  (pad "2" thru_hole oval (at 0 2.54 90) (size 1.7 1.7) (drill 1) (layers "*.Cu" "*.Mask") (remove_unused_layers no) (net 6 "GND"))
  (pad "3" thru_hole oval (at 0 5.08 90) (size 1.7 1.7) (drill 1) (layers "*.Cu" "*.Mask") (remove_unused_layers no) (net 6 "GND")))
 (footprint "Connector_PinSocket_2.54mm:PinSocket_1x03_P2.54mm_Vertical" (layer "F.Cu") (at 123 96.5 90)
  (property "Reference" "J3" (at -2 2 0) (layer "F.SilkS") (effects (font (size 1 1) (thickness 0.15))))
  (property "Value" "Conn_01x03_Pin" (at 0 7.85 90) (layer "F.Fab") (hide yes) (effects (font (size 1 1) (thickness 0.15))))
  (fp_line (start 1.33 -1.33) (end 1.33 0) (stroke (width 0.12) (type solid)) (layer "F.SilkS"))
  (fp_line (start 0 -1.33) (end 1.33 -1.33) (stroke (width 0.12) (type solid)) (layer "F.SilkS"))
  (fp_line (start 1.33 1.27) (end 1.33 6.41) (stroke (width 0.12) (type solid)) (layer "F.SilkS"))
  (fp_line (start -1.33 1.27) (end 1.33 1.27) (stroke (width 0.12) (type solid)) (layer "F.SilkS"))
  (fp_line (start -1.33 1.27) (end -1.33 6.41) (stroke (width 0.12) (type solid)) (layer "F.SilkS"))
  (fp_line (start -1.33 6.41) (end 1.33 6.41) (stroke (width 0.12) (type solid)) (layer "F.SilkS"))
  (pad "1" thru_hole rect (at 0 0 90) (size 1.7 1.7) (drill 1) (layers "*.Cu" "*.Mask") (remove_unused_layers no) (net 1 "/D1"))
  (pad "2" thru_hole oval (at 0 2.54 90) (size 1.7 1.7) (drill 1) (layers "*.Cu" "*.Mask") (remove_unused_layers no) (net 6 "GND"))
  (pad "3" thru_hole oval (at 0 5.08 90) (size 1.7 1.7) (drill 1) (layers "*.Cu" "*.Mask") (remove_unused_layers no) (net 6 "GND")))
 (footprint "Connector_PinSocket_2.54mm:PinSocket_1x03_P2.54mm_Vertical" (layer "F.Cu") (at 113.835 80.405 90)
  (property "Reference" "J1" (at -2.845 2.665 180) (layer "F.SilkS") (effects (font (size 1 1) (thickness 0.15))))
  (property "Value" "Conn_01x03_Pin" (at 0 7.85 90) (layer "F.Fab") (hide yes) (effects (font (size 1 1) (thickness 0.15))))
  (fp_line (start 1.33 -1.33) (end 1.33 0) (stroke (width 0.12) (type solid)) (layer "F.SilkS"))
  (fp_line (start 0 -1.33) (end 1.33 -1.33) (stroke (width 0.12) (type solid)) (layer "F.SilkS"))
  (fp_line (start 1.33 1.27) (end 1.33 6.41) (stroke (width 0.12) (type solid)) (layer "F.SilkS"))
  (fp_line (start -1.33 1.27) (end 1.33 1.27) (stroke (width 0.12) (type solid)) (layer "F.SilkS"))
  (fp_line (start -1.33 1.27) (end -1.33 6.41) (stroke (width 0.12) (type solid)) (layer "F.SilkS"))
  (fp_line (start -1.33 6.41) (end 1.33 6.41) (stroke (width 0.12) (type solid)) (layer "F.SilkS"))
  (pad "1" thru_hole rect (at 0 0 90) (size 1.7 1.7) (drill 1) (layers "*.Cu" "*.Mask") (remove_unused_layers no) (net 1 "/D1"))
  (pad "2" thru_hole oval (at 0 2.54 90) (size 1.7 1.7) (drill 1) (layers "*.Cu" "*.Mask") (remove_unused_layers no) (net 6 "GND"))
  (pad "3" thru_hole oval (at 0 5.08 90) (size 1.7 1.7) (drill 1) (layers "*.Cu" "*.Mask") (remove_unused_layers no) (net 6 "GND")))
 (gr_line (start 151 84) (end 151 70) (stroke (width 0.2) (type default)) (layer "B.Cu"))
 (gr_line (start 95 84) (end 165 84) (stroke (width 0.2) (type default)) (layer "B.Cu"))
 (gr_line (start 137 70) (end 137 84) (stroke (width 0.2) (type default)) (layer "B.Cu"))
 (gr_line (start 109 70) (end 109 84) (stroke (width 0.2) (type default)) (layer "B.Cu"))
 (gr_line (start 123 84) (end 123 70) (stroke (width 0.2) (type default)) (layer "B.Cu"))
 (gr_line (start 115 100) (end 115 84) (stroke (width 0.2) (type default)) (layer "B.Cu"))
 (gr_line (start 95 70) (end 165 70) (stroke (width 0.05) (type default)) (layer "Edge.Cuts"))
 (gr_line (start 95 84) (end 95 100) (stroke (width 0.05) (type default)) (layer "Edge.Cuts"))
 (gr_line (start 95 100) (end 135 100) (stroke (width 0.05) (type default)) (layer "Edge.Cuts"))
 (gr_line (start 135 100) (end 135 84) (stroke (width 0.05) (type default)) (layer "Edge.Cuts"))
 (gr_line (start 165 70) (end 165 84) (stroke (width 0.05) (type default)) (layer "Edge.Cuts"))
 (gr_line (start 165 84) (end 95 84) (stroke (width 0.05) (type default)) (layer "Edge.Cuts"))
 (gr_line (start 95 84) (end 95 70) (stroke (width 0.05) (type default)) (layer "Edge.Cuts"))
 (segment (start 121.5 80.25) (end 121.5 77.75) (width 1) (layer "B.Cu") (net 6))
 (segment (start 160.665 80.255) (end 163.095 80.255) (width 1) (layer "B.Cu") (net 6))
 (segment (start 116.375 80.405) (end 118.915 80.405) (width 1) (layer "B.Cu") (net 6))
 (segment (start 113.229671 96) (end 113.229671 94) (width 1) (layer "B.Cu") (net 6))
 (segment (start 125.54 96.5) (end 128.08 96.5) (width 1) (layer "B.Cu") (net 6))
 (segment (start 147.125 77.345) (end 148.625 77.345) (width 1) (layer "B.Cu") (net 6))
 (segment (start 118.915 80.405) (end 121.345 80.405) (width 1) (layer "B.Cu") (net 6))
 (segment (start 121 77.25) (end 121.5 77.75) (width 1) (layer "B.Cu") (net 6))
 (segment (start 148.97 80.5) (end 149.125 80.345) (width 1) (layer "B.Cu") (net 6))
 (segment (start 112.229671 93) (end 111.229671 93) (width 1) (layer "B.Cu") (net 6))
 (segment (start 163.095 80.255) (end 163.25 80.1) (width 1) (layer "B.Cu") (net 6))
 (segment (start 132.5 96.5) (end 133.5 95.5) (width 1) (layer "B.Cu") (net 6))
 (segment (start 113.229671 94) (end 112.229671 93) (width 1) (layer "B.Cu") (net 6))
 (segment (start 149.125 80.345) (end 149.125 77.845) (width 1) (layer "B.Cu") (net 6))
 (segment (start 133.5 95.5) (end 133.5 93.5) (width 1) (layer "B.Cu") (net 6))
 (segment (start 135.5 80.25) (end 135.5 77.75) (width 1) (layer "B.Cu") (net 6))
 (segment (start 106.5 77.5) (end 107 78) (width 1) (layer "B.Cu") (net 6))
 (segment (start 133.5 93.5) (end 132.5 92.5) (width 1) (layer "B.Cu") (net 6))
 (segment (start 106.845 80.655) (end 107 80.5) (width 1) (layer "B.Cu") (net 6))
 (segment (start 105.269671 97) (end 107.809671 97) (width 1) (layer "B.Cu") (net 6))
 (segment (start 132.915 80.405) (end 135.345 80.405) (width 1) (layer "B.Cu") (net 6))
 (segment (start 107 80.5) (end 107 78) (width 1) (layer "B.Cu") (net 6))
 (segment (start 146.54 80.5) (end 148.97 80.5) (width 1) (layer "B.Cu") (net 6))
 (segment (start 162.75 77.1) (end 163.25 77.6) (width 1) (layer "B.Cu") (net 6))
 (segment (start 105 77.5) (end 106.5 77.5) (width 1) (layer "B.Cu") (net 6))
 (segment (start 148.625 77.345) (end 149.125 77.845) (width 1) (layer "B.Cu") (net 6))
 (segment (start 121.345 80.405) (end 121.5 80.25) (width 1) (layer "B.Cu") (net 6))
 (segment (start 104.415 80.655) (end 106.845 80.655) (width 1) (layer "B.Cu") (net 6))
 (segment (start 119.5 77.25) (end 121 77.25) (width 1) (layer "B.Cu") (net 6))
 (segment (start 158.125 80.255) (end 160.665 80.255) (width 1) (layer "B.Cu") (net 6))
 (segment (start 112.229671 97) (end 113.229671 96) (width 1) (layer "B.Cu") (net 6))
 (segment (start 144 80.5) (end 146.54 80.5) (width 1) (layer "B.Cu") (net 6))
 (segment (start 163.25 80.1) (end 163.25 77.6) (width 1) (layer "B.Cu") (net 6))
 (segment (start 101.875 80.655) (end 104.415 80.655) (width 1) (layer "B.Cu") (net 6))
 (segment (start 133.5 77.25) (end 135 77.25) (width 1) (layer "B.Cu") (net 6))
 (segment (start 132.5 92.5) (end 131.5 92.5) (width 1) (layer "B.Cu") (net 6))
 (segment (start 128.08 96.5) (end 132.5 96.5) (width 1) (layer "B.Cu") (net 6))
 (segment (start 135 77.25) (end 135.5 77.75) (width 1) (layer "B.Cu") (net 6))
 (segment (start 161.25 77.1) (end 162.75 77.1) (width 1) (layer "B.Cu") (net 6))
 (segment (start 107.809671 97) (end 112.229671 97) (width 1) (layer "B.Cu") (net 6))
 (segment (start 130.375 80.405) (end 132.915 80.405) (width 1) (layer "B.Cu") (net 6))
 (segment (start 135.345 80.405) (end 135.5 80.25) (width 1) (layer "B.Cu") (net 6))
 (segment (start 152.75 78.6) (end 152.75 74.1) (width 0.6) (layer "B.Cu") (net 1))
 (segment (start 154.25 72.6) (end 154.75 72.6) (width 0.6) (layer "B.Cu") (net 1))
 (segment (start 97.729671 97) (end 96.729671 96) (width 0.6) (layer "B.Cu") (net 1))
 (segment (start 125 78.75) (end 125 74.25) (width 0.6) (layer "B.Cu") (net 1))
 (segment (start 102.729671 97) (end 97.729671 97) (width 0.6) (layer "B.Cu") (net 1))
 (segment (start 155.585 80.255) (end 154.405 80.255) (width 0.6) (layer "B.Cu") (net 1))
 (segment (start 111 78.75) (end 111 74.25) (width 0.6) (layer "B.Cu") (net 1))
 (segment (start 118 96.5) (end 117 95.5) (width 0.6) (layer "B.Cu") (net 1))
 (segment (start 138.625 74.345) (end 140.125 72.845) (width 0.6) (layer "B.Cu") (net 1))
 (segment (start 96.729671 90) (end 98.729671 88) (width 0.6) (layer "B.Cu") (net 1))
 (segment (start 125 74.25) (end 126.5 72.75) (width 0.6) (layer "B.Cu") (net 1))
 (segment (start 138.625 78.845) (end 138.625 74.345) (width 0.6) (layer "B.Cu") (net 1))
 (segment (start 140.28 80.5) (end 138.625 78.845) (width 0.6) (layer "B.Cu") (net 1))
 (segment (start 98.155 80.655) (end 96.5 79) (width 0.6) (layer "B.Cu") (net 1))
 (segment (start 126.655 80.405) (end 125 78.75) (width 0.6) (layer "B.Cu") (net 1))
 (segment (start 99.335 80.655) (end 98.155 80.655) (width 0.6) (layer "B.Cu") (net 1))
 (segment (start 141.46 80.5) (end 140.28 80.5) (width 0.6) (layer "B.Cu") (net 1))
 (segment (start 113.835 80.405) (end 112.655 80.405) (width 0.6) (layer "B.Cu") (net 1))
 (segment (start 126.5 72.75) (end 127 72.75) (width 0.6) (layer "B.Cu") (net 1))
 (segment (start 154.405 80.255) (end 152.75 78.6) (width 0.6) (layer "B.Cu") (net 1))
 (segment (start 111 74.25) (end 112.5 72.75) (width 0.6) (layer "B.Cu") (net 1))
 (segment (start 98 73) (end 98.5 73) (width 0.6) (layer "B.Cu") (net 1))
 (segment (start 112.5 72.75) (end 113 72.75) (width 0.6) (layer "B.Cu") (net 1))
 (segment (start 96.729671 96) (end 96.729671 90) (width 0.6) (layer "B.Cu") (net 1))
 (segment (start 96.5 79) (end 96.5 74.5) (width 0.6) (layer "B.Cu") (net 1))
 (segment (start 140.125 72.845) (end 140.625 72.845) (width 0.6) (layer "B.Cu") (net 1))
 (segment (start 152.75 74.1) (end 154.25 72.6) (width 0.6) (layer "B.Cu") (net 1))
 (segment (start 117 95.5) (end 117 89.5) (width 0.6) (layer "B.Cu") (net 1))
 (segment (start 127.835 80.405) (end 126.655 80.405) (width 0.6) (layer "B.Cu") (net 1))
 (segment (start 123 96.5) (end 118 96.5) (width 0.6) (layer "B.Cu") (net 1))
 (segment (start 112.655 80.405) (end 111 78.75) (width 0.6) (layer "B.Cu") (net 1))
 (segment (start 96.5 74.5) (end 98 73) (width 0.6) (layer "B.Cu") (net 1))
 (segment (start 117 89.5) (end 119 87.5) (width 0.6) (layer "B.Cu") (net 1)))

